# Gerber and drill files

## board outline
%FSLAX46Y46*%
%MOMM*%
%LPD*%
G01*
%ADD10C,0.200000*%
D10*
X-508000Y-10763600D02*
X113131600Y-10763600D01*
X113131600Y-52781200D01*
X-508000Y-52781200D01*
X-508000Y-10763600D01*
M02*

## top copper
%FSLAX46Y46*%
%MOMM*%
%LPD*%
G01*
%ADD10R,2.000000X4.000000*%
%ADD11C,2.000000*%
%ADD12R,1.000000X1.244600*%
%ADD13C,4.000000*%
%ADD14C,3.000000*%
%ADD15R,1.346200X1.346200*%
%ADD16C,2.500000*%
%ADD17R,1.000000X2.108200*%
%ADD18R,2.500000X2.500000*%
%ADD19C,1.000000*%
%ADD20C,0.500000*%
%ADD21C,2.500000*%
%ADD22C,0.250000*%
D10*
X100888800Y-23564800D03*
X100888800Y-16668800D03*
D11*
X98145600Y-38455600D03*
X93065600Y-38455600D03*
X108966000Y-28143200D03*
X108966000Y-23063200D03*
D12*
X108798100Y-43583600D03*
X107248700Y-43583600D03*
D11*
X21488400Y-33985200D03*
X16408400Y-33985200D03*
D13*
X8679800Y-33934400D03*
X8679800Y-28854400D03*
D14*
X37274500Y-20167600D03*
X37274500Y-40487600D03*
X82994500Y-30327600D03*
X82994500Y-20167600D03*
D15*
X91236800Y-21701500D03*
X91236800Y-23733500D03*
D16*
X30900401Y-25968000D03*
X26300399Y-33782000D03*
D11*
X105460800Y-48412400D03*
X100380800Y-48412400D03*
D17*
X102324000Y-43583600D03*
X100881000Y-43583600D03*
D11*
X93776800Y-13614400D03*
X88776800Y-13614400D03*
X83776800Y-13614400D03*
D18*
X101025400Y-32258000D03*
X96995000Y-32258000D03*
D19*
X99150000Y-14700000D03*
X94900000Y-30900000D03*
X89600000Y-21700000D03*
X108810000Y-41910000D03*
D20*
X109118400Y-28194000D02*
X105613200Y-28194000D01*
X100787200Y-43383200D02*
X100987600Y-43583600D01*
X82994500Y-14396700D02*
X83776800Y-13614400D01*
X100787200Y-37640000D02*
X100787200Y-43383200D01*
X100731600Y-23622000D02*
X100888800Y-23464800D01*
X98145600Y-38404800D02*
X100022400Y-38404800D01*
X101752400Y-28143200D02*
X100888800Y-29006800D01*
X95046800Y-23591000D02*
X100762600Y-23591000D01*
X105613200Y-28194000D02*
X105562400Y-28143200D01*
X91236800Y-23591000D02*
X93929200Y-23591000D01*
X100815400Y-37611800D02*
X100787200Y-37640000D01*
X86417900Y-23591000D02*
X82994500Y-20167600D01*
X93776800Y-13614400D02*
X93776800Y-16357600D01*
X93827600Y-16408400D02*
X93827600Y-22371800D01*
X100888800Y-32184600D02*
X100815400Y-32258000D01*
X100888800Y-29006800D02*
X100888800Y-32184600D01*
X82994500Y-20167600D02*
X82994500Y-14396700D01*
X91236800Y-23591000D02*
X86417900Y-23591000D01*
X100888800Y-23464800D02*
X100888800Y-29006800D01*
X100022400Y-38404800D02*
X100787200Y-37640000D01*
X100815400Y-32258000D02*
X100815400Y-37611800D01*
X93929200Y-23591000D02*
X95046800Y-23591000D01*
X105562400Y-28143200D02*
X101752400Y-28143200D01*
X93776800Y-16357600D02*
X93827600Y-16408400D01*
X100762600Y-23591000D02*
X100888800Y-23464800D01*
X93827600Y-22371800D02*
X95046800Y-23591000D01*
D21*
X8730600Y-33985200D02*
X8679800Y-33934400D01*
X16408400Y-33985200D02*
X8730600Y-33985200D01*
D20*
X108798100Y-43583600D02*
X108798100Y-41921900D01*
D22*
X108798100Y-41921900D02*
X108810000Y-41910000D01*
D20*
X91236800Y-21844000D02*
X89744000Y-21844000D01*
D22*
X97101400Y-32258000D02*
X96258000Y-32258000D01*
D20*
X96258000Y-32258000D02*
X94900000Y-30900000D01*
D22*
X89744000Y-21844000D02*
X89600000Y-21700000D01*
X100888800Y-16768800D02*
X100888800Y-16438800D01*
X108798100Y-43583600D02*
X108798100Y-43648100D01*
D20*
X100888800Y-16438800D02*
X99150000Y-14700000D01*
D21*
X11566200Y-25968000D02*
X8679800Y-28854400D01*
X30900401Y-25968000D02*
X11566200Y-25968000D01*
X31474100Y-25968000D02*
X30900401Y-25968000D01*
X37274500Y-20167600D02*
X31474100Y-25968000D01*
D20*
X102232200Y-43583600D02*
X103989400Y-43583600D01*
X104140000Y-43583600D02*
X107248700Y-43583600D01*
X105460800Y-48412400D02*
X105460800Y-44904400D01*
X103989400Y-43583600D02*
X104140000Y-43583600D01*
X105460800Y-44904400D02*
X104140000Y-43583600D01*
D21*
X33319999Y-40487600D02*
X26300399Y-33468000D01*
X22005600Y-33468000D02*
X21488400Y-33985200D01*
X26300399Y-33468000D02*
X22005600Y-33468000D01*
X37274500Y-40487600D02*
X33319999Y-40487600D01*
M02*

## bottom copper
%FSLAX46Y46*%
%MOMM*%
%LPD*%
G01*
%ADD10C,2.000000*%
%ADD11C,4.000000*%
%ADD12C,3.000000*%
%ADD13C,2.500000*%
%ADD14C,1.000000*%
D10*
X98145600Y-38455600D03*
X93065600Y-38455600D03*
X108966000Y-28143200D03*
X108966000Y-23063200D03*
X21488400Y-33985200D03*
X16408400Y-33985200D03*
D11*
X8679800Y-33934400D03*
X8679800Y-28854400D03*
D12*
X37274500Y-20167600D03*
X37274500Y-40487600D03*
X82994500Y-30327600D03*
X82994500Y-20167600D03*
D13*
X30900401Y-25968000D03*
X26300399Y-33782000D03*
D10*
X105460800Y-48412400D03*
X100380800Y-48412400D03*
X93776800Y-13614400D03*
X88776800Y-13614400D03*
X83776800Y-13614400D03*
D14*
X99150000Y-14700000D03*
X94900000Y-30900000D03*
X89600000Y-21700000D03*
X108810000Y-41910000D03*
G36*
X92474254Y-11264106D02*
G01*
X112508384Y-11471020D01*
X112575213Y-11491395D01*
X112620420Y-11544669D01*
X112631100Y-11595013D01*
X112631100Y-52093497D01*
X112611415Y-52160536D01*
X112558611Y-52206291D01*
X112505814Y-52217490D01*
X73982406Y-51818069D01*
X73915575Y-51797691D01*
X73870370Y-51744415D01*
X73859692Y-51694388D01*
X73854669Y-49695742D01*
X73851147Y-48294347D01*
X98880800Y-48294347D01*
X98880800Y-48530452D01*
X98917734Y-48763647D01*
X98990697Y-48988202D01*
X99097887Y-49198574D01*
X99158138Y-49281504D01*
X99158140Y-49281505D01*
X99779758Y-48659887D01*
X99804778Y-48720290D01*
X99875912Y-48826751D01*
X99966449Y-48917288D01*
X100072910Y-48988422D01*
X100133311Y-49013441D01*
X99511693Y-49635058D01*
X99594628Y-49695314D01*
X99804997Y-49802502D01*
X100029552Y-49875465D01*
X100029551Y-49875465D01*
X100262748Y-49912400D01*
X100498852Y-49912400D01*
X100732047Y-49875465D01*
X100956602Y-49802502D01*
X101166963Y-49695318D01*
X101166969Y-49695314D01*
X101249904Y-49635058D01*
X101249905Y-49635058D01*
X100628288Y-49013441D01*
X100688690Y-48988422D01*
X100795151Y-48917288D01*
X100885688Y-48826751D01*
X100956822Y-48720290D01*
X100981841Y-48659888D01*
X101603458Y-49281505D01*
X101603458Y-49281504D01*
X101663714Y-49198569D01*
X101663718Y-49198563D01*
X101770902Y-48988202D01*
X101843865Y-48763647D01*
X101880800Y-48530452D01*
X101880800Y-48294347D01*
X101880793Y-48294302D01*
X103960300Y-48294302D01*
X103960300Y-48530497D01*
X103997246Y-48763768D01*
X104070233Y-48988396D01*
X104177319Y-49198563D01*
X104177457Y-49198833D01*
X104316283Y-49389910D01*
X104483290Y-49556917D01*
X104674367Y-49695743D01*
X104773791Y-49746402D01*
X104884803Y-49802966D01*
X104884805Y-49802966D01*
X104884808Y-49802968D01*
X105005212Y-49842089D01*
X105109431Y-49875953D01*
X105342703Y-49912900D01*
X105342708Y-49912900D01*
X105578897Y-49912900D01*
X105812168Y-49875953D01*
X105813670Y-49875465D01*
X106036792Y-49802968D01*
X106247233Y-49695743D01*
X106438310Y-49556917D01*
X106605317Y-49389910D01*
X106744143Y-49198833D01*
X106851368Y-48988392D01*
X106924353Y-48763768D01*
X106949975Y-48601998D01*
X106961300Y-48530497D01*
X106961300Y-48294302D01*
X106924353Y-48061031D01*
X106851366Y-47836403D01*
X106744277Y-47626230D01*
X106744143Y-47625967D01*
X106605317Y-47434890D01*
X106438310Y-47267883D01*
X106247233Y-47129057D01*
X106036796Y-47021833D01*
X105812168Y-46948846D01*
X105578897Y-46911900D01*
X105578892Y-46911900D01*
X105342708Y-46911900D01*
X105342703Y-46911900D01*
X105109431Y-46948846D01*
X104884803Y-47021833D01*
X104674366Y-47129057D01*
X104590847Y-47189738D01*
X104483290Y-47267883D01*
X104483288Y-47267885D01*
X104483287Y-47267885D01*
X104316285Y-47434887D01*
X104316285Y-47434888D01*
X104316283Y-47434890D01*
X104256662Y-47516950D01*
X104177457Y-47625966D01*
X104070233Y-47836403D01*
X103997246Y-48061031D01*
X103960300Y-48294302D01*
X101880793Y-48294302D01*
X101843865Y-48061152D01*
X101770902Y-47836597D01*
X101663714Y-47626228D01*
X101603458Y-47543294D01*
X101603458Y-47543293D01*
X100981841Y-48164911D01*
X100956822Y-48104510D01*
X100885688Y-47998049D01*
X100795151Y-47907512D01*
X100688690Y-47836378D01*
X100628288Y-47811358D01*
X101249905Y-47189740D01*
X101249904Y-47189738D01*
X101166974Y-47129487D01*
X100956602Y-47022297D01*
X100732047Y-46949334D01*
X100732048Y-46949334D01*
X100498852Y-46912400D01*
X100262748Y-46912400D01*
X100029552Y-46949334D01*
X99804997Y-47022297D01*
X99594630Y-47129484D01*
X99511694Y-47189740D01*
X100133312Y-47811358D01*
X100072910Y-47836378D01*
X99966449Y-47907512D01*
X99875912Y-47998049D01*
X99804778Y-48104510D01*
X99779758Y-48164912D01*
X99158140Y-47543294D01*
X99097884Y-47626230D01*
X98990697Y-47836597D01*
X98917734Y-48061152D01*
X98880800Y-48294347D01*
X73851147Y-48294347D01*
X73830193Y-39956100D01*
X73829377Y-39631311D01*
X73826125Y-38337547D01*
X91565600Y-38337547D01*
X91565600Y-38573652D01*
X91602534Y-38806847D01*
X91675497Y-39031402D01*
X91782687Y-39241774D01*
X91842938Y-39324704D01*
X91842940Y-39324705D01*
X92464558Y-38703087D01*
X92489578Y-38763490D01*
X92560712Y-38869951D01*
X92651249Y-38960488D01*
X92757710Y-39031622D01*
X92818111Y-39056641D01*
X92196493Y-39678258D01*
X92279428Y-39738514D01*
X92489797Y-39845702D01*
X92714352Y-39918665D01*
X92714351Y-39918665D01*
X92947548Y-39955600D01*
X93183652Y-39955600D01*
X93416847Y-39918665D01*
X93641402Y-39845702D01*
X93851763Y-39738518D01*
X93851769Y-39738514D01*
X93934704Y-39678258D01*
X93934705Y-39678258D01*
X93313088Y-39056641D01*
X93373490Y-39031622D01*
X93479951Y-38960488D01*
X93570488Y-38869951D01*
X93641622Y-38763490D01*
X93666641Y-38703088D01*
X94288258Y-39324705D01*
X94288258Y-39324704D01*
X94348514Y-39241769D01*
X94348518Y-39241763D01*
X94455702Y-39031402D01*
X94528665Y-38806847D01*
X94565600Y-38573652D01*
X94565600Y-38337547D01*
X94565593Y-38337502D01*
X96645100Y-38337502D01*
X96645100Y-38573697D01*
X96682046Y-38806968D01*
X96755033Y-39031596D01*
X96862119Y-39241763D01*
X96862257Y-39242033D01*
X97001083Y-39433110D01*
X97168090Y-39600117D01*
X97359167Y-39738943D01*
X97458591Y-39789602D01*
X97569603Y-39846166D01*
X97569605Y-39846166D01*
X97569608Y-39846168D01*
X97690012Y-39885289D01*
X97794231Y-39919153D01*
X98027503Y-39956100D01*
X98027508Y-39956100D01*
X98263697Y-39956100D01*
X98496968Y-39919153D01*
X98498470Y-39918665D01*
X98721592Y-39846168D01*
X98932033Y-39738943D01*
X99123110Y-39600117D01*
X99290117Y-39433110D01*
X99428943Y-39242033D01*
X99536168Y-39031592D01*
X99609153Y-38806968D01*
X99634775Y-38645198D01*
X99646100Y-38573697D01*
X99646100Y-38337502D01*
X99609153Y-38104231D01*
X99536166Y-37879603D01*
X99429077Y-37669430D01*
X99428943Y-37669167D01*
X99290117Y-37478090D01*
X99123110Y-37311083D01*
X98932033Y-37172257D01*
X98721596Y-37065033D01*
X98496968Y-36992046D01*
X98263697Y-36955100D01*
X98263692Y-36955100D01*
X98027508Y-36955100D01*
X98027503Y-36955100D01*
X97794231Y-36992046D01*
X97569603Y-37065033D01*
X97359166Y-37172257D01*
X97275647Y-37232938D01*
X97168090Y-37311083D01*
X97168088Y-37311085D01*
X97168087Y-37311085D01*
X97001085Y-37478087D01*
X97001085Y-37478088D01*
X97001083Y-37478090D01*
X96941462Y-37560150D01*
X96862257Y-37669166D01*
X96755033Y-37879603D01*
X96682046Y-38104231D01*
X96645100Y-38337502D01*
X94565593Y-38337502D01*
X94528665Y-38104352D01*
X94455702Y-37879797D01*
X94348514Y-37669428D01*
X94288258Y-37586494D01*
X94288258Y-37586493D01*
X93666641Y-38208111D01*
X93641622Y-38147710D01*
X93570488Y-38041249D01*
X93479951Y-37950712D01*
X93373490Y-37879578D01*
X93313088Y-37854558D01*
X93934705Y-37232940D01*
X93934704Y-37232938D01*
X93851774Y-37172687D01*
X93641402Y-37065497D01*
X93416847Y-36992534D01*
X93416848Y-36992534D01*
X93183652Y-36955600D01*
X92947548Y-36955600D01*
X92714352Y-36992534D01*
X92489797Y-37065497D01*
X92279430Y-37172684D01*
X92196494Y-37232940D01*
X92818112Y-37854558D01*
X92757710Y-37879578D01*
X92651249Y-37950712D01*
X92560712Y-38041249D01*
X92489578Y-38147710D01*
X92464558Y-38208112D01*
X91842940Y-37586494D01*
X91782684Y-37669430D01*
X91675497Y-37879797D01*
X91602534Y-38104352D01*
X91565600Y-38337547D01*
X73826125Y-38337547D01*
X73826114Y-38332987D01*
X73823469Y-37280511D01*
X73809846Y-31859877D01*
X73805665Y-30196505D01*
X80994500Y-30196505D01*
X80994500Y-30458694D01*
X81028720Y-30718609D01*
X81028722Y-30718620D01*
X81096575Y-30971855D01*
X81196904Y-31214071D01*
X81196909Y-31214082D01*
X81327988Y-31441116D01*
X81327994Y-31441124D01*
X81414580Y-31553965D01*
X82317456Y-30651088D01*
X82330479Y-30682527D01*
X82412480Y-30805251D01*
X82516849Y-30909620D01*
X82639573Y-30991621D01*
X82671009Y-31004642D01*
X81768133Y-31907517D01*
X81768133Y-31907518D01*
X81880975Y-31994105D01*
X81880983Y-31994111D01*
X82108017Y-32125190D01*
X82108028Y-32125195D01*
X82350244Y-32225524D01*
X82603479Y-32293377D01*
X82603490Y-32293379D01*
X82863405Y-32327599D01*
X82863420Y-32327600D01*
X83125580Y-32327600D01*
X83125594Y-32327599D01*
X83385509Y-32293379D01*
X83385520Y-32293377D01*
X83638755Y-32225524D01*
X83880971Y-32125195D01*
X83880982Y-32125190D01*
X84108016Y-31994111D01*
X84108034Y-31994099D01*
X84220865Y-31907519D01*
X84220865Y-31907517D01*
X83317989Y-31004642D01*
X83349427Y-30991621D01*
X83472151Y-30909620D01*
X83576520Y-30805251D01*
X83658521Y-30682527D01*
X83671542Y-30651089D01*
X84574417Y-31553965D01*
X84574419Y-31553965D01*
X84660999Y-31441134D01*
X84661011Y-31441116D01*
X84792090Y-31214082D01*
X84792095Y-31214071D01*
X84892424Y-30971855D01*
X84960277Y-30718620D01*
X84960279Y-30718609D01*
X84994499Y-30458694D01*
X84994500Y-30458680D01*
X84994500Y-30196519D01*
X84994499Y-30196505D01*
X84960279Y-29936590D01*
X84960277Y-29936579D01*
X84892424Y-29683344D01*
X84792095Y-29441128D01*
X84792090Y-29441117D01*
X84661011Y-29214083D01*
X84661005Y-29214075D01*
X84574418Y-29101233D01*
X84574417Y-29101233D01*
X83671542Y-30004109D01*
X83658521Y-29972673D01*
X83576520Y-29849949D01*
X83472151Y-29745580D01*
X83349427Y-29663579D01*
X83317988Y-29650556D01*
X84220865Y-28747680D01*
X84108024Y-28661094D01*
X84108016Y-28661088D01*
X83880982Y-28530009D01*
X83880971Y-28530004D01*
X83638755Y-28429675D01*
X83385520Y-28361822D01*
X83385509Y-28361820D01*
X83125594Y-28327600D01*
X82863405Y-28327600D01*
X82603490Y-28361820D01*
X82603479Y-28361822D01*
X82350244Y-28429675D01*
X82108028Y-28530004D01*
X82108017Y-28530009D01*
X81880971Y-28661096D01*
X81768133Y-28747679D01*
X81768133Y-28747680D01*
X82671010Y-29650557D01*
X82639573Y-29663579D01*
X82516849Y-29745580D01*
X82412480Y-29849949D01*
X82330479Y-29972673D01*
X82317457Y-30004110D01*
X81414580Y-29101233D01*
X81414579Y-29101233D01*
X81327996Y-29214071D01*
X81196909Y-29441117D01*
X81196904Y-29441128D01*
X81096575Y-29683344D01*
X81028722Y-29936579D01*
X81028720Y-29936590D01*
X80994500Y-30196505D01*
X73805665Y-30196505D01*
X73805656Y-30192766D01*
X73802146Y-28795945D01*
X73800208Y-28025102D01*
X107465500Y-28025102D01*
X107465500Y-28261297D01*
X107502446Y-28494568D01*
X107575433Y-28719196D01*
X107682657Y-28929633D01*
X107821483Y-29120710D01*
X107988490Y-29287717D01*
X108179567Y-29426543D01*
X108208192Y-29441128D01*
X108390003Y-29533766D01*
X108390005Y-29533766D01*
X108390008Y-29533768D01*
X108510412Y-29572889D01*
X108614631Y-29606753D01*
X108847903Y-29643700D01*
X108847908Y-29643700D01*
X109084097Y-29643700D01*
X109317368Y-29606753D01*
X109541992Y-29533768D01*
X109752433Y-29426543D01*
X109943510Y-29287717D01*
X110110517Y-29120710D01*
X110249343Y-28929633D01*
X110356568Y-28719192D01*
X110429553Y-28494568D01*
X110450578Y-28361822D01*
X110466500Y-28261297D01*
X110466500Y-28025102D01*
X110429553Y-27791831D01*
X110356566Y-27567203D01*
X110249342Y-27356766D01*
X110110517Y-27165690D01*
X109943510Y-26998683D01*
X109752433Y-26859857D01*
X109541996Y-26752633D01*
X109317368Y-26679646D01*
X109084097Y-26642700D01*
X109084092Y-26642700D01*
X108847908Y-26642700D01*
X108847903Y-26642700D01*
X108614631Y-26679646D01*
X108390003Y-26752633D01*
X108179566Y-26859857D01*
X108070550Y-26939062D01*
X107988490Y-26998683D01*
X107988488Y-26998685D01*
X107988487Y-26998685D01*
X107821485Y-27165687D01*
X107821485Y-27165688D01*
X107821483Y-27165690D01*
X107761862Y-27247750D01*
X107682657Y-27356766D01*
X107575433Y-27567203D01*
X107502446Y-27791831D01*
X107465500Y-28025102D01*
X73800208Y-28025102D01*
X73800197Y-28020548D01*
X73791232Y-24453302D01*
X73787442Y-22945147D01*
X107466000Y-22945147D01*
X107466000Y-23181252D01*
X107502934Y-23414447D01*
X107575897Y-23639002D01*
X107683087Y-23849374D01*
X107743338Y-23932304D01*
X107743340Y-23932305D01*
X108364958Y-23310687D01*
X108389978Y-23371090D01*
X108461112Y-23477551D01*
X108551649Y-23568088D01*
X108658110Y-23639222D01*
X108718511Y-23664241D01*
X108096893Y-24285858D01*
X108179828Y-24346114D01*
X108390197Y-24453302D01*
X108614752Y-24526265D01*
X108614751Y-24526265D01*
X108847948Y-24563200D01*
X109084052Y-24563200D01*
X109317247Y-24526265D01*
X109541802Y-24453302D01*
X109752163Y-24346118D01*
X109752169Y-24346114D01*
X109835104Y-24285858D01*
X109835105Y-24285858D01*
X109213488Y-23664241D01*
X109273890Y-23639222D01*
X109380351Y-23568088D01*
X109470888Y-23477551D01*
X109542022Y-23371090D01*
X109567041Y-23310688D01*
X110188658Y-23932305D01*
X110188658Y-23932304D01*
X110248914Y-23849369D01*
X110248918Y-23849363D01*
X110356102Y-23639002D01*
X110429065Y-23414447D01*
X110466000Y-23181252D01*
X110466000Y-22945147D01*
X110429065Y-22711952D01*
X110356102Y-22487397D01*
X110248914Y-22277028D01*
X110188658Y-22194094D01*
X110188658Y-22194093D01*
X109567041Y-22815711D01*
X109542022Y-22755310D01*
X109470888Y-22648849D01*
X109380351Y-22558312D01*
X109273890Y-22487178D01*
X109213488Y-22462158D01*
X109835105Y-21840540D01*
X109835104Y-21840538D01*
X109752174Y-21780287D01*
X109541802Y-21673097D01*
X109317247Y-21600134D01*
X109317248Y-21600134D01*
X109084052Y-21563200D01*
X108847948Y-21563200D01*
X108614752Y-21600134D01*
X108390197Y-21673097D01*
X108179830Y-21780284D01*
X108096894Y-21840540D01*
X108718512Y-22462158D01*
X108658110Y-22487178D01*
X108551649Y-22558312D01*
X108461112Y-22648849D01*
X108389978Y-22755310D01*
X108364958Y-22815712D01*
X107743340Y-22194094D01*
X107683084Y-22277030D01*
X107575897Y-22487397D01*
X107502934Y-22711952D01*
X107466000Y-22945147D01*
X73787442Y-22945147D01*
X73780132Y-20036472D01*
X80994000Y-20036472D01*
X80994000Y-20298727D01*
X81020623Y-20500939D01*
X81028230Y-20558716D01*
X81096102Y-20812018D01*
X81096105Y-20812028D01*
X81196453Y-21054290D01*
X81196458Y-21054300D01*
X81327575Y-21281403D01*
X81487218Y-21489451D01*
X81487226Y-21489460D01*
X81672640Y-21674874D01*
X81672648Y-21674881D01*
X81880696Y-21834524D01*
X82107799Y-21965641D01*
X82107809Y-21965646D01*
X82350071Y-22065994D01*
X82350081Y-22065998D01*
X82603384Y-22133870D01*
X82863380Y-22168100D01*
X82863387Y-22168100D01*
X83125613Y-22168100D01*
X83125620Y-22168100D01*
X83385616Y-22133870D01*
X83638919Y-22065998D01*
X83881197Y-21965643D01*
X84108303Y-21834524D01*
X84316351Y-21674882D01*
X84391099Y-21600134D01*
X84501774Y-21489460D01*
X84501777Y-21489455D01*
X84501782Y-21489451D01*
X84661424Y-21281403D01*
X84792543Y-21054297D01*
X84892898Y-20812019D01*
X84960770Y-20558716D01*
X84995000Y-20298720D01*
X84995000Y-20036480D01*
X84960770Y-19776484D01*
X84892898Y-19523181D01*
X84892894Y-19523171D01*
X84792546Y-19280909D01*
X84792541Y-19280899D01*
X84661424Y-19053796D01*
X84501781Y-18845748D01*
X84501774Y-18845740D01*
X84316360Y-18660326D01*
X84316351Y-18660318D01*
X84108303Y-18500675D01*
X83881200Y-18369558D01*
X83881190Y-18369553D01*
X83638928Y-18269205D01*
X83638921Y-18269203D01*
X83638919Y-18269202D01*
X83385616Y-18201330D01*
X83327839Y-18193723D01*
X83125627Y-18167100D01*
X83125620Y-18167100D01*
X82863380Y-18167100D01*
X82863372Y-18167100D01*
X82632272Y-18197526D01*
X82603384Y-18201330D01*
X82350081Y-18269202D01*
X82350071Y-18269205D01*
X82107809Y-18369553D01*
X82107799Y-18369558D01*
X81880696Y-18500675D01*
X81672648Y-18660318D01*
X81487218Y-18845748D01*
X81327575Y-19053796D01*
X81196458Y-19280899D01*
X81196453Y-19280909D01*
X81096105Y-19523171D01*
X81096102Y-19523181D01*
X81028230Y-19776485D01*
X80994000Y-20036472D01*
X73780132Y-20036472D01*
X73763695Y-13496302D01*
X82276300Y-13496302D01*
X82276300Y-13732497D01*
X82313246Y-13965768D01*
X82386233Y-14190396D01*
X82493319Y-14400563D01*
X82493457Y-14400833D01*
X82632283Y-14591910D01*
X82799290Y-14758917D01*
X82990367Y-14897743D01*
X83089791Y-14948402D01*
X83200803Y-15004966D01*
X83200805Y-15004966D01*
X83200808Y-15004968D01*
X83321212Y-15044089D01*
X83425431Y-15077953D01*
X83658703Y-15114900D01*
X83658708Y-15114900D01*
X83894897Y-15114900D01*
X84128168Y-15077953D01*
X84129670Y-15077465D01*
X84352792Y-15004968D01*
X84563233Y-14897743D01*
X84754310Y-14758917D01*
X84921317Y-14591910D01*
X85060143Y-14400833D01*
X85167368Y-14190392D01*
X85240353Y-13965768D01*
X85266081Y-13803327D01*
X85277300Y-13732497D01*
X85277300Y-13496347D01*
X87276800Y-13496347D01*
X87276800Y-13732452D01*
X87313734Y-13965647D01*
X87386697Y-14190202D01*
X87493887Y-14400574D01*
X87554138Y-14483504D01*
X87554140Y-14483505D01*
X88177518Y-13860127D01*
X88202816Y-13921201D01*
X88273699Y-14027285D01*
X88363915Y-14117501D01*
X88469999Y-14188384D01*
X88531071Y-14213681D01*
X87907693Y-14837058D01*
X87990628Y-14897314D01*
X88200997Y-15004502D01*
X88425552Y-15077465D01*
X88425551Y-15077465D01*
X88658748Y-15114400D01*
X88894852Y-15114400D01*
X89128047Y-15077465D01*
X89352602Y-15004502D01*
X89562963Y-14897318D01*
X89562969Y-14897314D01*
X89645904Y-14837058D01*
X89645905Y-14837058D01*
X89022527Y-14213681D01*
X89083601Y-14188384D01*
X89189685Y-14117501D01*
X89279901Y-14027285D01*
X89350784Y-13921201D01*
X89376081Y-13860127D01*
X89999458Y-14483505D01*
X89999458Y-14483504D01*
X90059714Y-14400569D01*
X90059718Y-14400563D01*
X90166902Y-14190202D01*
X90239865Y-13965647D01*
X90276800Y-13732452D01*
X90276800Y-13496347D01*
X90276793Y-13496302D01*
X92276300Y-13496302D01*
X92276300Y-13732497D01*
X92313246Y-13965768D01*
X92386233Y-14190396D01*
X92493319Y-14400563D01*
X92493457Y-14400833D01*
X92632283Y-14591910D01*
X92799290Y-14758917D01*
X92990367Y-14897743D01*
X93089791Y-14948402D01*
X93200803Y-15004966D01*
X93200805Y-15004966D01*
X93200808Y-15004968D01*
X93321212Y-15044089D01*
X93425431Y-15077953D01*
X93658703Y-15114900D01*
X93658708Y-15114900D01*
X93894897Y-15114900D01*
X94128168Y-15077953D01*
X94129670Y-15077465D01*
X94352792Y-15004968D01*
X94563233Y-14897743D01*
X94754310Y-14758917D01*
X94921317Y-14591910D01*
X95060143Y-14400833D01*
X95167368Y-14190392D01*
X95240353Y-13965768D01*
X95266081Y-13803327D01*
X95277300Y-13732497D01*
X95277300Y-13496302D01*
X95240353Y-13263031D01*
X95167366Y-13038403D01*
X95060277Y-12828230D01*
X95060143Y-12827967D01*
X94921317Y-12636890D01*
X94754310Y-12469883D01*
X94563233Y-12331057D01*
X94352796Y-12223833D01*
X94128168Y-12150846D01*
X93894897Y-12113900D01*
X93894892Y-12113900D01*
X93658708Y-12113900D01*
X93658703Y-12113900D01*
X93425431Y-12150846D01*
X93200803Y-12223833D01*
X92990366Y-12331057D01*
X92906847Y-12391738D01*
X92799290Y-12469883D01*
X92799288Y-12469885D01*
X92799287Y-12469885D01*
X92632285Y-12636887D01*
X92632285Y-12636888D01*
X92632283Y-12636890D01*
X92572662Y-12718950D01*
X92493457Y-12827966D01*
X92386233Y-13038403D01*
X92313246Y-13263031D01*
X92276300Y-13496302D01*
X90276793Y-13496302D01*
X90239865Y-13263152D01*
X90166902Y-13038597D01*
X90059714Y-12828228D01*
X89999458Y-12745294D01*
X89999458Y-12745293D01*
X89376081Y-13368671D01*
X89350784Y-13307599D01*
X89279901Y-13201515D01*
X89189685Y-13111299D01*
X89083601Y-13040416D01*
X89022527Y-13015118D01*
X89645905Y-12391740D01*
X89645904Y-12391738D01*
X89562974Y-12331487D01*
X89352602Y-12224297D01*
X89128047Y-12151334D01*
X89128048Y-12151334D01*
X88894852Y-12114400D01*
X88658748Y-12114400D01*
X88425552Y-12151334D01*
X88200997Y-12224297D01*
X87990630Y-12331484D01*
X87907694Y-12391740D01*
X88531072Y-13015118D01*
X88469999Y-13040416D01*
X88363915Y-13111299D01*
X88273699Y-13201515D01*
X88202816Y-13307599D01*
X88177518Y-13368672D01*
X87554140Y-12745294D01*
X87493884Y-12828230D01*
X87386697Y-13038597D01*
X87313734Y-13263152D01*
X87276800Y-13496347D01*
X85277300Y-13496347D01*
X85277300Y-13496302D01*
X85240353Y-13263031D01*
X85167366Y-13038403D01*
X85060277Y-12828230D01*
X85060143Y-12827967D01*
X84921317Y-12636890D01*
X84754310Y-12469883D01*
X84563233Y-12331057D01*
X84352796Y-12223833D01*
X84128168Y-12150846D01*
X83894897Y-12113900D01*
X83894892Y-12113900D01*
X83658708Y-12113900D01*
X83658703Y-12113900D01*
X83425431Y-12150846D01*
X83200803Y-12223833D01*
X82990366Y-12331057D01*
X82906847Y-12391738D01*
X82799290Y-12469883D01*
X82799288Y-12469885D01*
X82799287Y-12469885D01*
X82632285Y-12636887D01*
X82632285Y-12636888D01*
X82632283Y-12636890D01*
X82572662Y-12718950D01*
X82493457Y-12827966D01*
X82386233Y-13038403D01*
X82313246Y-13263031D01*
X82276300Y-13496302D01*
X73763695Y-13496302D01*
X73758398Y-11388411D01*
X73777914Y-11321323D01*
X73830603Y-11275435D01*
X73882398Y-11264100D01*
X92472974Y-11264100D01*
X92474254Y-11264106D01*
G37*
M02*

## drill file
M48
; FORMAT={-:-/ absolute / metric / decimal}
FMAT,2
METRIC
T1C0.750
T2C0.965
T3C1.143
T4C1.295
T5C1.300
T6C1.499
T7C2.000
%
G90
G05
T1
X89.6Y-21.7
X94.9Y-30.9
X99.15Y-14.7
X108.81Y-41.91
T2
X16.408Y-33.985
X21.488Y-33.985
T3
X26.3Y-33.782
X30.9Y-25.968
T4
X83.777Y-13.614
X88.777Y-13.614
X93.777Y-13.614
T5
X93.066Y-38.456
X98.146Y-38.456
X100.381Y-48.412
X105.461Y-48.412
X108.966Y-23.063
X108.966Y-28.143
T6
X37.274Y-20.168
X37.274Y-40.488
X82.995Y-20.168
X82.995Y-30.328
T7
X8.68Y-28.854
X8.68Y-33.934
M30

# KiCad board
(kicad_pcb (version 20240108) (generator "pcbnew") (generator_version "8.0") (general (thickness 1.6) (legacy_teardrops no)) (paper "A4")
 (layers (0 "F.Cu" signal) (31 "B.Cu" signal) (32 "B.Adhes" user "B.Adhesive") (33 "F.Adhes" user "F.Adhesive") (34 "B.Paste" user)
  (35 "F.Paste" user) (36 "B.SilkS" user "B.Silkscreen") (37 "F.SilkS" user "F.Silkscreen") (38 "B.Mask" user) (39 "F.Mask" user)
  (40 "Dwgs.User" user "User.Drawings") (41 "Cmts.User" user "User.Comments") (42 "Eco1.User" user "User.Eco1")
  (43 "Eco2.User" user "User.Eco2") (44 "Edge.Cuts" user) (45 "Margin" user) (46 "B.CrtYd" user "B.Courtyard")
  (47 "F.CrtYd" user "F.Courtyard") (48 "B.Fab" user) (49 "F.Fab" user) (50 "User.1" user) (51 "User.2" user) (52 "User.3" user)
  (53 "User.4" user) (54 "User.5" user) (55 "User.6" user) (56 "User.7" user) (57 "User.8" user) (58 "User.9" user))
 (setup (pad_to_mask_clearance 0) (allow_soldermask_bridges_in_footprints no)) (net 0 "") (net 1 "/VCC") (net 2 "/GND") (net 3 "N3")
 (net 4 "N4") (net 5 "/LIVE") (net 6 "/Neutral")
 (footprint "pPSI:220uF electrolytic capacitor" (layer "F.Cu") (at 100.8888 20.1168 90)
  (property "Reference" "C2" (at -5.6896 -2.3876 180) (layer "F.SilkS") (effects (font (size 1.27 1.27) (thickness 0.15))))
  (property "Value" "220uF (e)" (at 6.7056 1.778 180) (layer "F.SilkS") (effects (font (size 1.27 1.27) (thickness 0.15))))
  (pad "1" smd rect (at -3.448 0 90) (size 4 2) (layers "F.Cu" "F.Paste" "F.Mask") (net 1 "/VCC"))
  (pad "2" smd rect (at 3.448 0 90) (size 4 2) (layers "F.Cu" "F.Paste" "F.Mask") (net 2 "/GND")))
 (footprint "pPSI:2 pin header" (layer "F.Cu") (at 98.1456 38.4556 180)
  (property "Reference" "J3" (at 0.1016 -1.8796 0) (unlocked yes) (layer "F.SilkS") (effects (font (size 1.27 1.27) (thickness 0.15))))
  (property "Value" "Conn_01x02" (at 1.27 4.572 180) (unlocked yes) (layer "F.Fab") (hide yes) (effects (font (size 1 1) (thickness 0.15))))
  (pad "1" thru_hole circle (at 0 0 180) (size 2 2) (drill 1.3) (layers "*.Cu" "*.Mask") (remove_unused_layers no) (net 1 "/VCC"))
  (pad "2" thru_hole circle (at 5.08 0 180) (size 2 2) (drill 1.3) (layers "*.Cu" "*.Mask") (remove_unused_layers no) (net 2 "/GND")))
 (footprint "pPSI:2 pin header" (layer "F.Cu") (at 108.966 28.1432 90)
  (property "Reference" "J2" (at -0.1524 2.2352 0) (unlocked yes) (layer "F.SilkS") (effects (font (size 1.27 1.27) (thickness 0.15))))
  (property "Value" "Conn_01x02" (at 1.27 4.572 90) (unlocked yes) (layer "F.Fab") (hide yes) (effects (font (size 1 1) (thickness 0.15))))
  (pad "1" thru_hole circle (at 0 0 90) (size 2 2) (drill 1.3) (layers "*.Cu" "*.Mask") (remove_unused_layers no) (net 1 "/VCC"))
  (pad "2" thru_hole circle (at 5.08 0 90) (size 2 2) (drill 1.3) (layers "*.Cu" "*.Mask") (remove_unused_layers no) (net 2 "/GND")))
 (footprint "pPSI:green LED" (layer "F.Cu") (at 108.0234 43.5836 180)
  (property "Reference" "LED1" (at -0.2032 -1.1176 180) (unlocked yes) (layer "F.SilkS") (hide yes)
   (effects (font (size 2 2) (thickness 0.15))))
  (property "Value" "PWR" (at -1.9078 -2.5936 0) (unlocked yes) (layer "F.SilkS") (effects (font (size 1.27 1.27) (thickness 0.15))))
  (pad "1" smd rect (at -0.7747 0 180) (size 1 1.2446) (layers "F.Cu" "F.Paste" "F.Mask") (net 2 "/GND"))
  (pad "2" smd rect (at 0.7747 0 180) (size 1 1.2446) (layers "F.Cu" "F.Paste" "F.Mask") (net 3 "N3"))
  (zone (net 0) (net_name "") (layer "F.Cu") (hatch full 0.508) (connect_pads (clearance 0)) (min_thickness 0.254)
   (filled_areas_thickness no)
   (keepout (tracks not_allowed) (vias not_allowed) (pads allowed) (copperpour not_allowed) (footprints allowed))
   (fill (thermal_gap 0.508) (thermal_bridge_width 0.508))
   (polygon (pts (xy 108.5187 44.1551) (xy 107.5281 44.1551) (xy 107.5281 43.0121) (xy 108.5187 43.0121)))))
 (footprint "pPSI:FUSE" (layer "F.Cu") (at 21.4884 33.9852 180)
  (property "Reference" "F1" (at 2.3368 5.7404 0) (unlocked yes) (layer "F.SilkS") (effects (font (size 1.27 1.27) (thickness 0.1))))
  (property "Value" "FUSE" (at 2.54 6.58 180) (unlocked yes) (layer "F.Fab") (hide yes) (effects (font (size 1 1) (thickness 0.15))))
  (pad "1" thru_hole circle (at 0 0 180) (size 2 2) (drill 0.9652) (layers "*.Cu" "*.Mask") (remove_unused_layers no) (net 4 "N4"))
  (pad "2" thru_hole circle (at 5.08 0 180) (size 2 2) (drill 0.9652) (layers "*.Cu" "*.Mask") (remove_unused_layers no) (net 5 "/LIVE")))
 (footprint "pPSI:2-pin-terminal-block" (layer "F.Cu") (at 8.6798 33.9344 90)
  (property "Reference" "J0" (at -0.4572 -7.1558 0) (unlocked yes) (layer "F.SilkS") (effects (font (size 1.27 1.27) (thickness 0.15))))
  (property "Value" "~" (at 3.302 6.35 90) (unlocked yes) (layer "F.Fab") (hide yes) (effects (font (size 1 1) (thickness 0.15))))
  (pad "1" thru_hole circle (at 0 0 90) (size 4 4) (drill 2) (layers "*.Cu" "*.Mask") (remove_unused_layers no) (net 5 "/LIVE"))
  (pad "2" thru_hole circle (at 5.08 0 90) (size 4 4) (drill 2) (layers "*.Cu" "*.Mask") (remove_unused_layers no) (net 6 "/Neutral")))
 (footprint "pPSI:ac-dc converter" (layer "F.Cu") (at 37.2745 20.1676)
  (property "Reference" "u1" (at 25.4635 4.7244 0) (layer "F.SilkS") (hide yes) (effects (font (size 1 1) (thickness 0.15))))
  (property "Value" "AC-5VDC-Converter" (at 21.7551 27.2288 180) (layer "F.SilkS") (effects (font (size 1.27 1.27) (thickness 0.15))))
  (pad "1" thru_hole circle (at 0 0) (size 3 3) (drill 1.4986) (layers "*.Cu" "*.Mask") (remove_unused_layers no) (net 6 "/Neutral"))
  (pad "2" thru_hole circle (at 0 20.32) (size 3 3) (drill 1.4986) (layers "*.Cu" "*.Mask") (remove_unused_layers no) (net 4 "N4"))
  (pad "3" thru_hole circle (at 45.72 10.16) (size 3 3) (drill 1.4986) (layers "*.Cu" "*.Mask") (remove_unused_layers no) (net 2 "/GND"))
  (pad "4" thru_hole circle (at 45.72 0) (size 3 3) (drill 1.4986) (layers "*.Cu" "*.Mask") (remove_unused_layers no) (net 1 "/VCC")))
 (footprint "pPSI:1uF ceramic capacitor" (layer "F.Cu") (at 91.2368 22.7175 -90)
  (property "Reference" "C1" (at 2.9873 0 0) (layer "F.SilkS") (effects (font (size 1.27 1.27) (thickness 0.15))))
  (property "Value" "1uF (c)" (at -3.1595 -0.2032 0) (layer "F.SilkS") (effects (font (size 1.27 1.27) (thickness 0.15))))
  (pad "1" smd rect (at -1.016 0 270) (size 1.3462 1.3462) (layers "F.Cu" "F.Paste" "F.Mask") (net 2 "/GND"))
  (pad "2" smd rect (at 1.016 0 270) (size 1.3462 1.3462) (layers "F.Cu" "F.Paste" "F.Mask") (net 1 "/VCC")))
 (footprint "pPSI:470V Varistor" (layer "F.Cu") (at 28.6004 29.718 -90)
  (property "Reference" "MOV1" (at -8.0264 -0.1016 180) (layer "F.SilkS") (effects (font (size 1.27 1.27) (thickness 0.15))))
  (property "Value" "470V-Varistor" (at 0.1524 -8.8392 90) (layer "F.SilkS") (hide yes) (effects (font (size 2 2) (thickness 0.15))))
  (pad "1" thru_hole circle (at -3.75 -2.300001 270) (size 2.5 2.5) (drill 1.143) (layers "*.Cu" "*.Mask") (remove_unused_layers no)
   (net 6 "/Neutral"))
  (pad "2" thru_hole circle (at 4.064 2.300001 270) (size 2.5 2.5) (drill 1.143) (layers "*.Cu" "*.Mask") (remove_unused_layers no)
   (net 4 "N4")))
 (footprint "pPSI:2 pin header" (layer "F.Cu") (at 105.4608 48.4124 180)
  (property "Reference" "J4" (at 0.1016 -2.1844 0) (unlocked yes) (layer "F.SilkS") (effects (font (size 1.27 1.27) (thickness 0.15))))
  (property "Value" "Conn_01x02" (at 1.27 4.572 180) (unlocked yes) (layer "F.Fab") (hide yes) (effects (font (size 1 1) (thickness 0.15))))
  (pad "1" thru_hole circle (at 0 0 180) (size 2 2) (drill 1.3) (layers "*.Cu" "*.Mask") (remove_unused_layers no) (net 3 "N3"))
  (pad "2" thru_hole circle (at 5.08 0 180) (size 2 2) (drill 1.3) (layers "*.Cu" "*.Mask") (remove_unused_layers no) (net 2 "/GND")))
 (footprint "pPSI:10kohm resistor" (layer "F.Cu") (at 101.6099 43.5836 180)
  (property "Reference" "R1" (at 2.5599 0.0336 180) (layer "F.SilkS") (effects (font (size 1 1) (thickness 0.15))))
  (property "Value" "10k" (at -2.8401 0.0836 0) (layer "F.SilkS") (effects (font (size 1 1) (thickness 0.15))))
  (pad "1" smd rect (at -0.7141 0 180) (size 1 2.1082) (layers "F.Cu" "F.Paste" "F.Mask") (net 3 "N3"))
  (pad "2" smd rect (at 0.7289 0 180) (size 1 2.1082) (layers "F.Cu" "F.Paste" "F.Mask") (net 1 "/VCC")))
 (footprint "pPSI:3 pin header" (layer "F.Cu") (at 93.7768 13.6144 180)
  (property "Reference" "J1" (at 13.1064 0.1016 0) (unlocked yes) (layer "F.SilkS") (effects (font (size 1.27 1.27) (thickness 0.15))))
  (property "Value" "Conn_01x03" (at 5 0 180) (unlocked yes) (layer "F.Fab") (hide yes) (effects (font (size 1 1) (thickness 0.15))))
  (pad "1" thru_hole circle (at 0 0 180) (size 2 2) (drill 1.2954) (layers "*.Cu" "*.Mask") (remove_unused_layers no) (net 1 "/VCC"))
  (pad "2" thru_hole circle (at 5 0 180) (size 2 2) (drill 1.2954) (layers "*.Cu" "*.Mask") (remove_unused_layers no) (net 2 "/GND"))
  (pad "3" thru_hole circle (at 10 0 180) (size 2 2) (drill 1.2954) (layers "*.Cu" "*.Mask") (remove_unused_layers no) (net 1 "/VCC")))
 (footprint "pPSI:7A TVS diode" (layer "F.Cu") (at 98.9584 32.258 180)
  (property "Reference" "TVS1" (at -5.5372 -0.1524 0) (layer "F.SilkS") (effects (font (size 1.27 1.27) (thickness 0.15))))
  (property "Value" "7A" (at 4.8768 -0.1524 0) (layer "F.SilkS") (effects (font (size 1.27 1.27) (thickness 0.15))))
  (pad "1" smd rect (at -2.067 0 270) (size 2.5 2.5) (layers "F.Cu" "F.Paste" "F.Mask") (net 1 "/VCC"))
  (pad "2" smd rect (at 1.9634 0 270) (size 2.5 2.5) (layers "F.Cu" "F.Paste" "F.Mask") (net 2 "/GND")))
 (gr_rect (start -0.508 10.7636) (end 113.1316 52.7812) (stroke (width 0.2) (type default)) (fill none) (layer "Edge.Cuts"))
 (segment (start 109.1184 28.194) (end 105.6132 28.194) (width 0.5) (layer "F.Cu") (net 1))
 (segment (start 100.7872 43.3832) (end 100.9876 43.5836) (width 0.5) (layer "F.Cu") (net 1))
 (segment (start 82.9945 14.3967) (end 83.7768 13.6144) (width 0.5) (layer "F.Cu") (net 1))
 (segment (start 100.7872 37.64) (end 100.7872 43.3832) (width 0.5) (layer "F.Cu") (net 1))
 (segment (start 100.7316 23.622) (end 100.8888 23.4648) (width 0.5) (layer "F.Cu") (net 1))
 (segment (start 98.1456 38.4048) (end 100.0224 38.4048) (width 0.5) (layer "F.Cu") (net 1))
 (segment (start 101.7524 28.1432) (end 100.8888 29.0068) (width 0.5) (layer "F.Cu") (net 1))
 (segment (start 95.0468 23.591) (end 100.7626 23.591) (width 0.5) (layer "F.Cu") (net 1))
 (segment (start 105.6132 28.194) (end 105.5624 28.1432) (width 0.5) (layer "F.Cu") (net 1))
 (segment (start 91.2368 23.591) (end 93.9292 23.591) (width 0.5) (layer "F.Cu") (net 1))
 (segment (start 100.8154 37.6118) (end 100.7872 37.64) (width 0.5) (layer "F.Cu") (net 1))
 (segment (start 86.4179 23.591) (end 82.9945 20.1676) (width 0.5) (layer "F.Cu") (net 1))
 (segment (start 93.7768 13.6144) (end 93.7768 16.3576) (width 0.5) (layer "F.Cu") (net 1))
 (segment (start 93.8276 16.4084) (end 93.8276 22.3718) (width 0.5) (layer "F.Cu") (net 1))
 (segment (start 100.8888 32.1846) (end 100.8154 32.258) (width 0.5) (layer "F.Cu") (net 1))
 (segment (start 100.8888 29.0068) (end 100.8888 32.1846) (width 0.5) (layer "F.Cu") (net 1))
 (segment (start 82.9945 20.1676) (end 82.9945 14.3967) (width 0.5) (layer "F.Cu") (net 1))
 (segment (start 91.2368 23.591) (end 86.4179 23.591) (width 0.5) (layer "F.Cu") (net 1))
 (segment (start 100.8888 23.4648) (end 100.8888 29.0068) (width 0.5) (layer "F.Cu") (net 1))
 (segment (start 100.0224 38.4048) (end 100.7872 37.64) (width 0.5) (layer "F.Cu") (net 1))
 (segment (start 100.8154 32.258) (end 100.8154 37.6118) (width 0.5) (layer "F.Cu") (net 1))
 (segment (start 93.9292 23.591) (end 95.0468 23.591) (width 0.5) (layer "F.Cu") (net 1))
 (segment (start 105.5624 28.1432) (end 101.7524 28.1432) (width 0.5) (layer "F.Cu") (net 1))
 (segment (start 93.7768 16.3576) (end 93.8276 16.4084) (width 0.5) (layer "F.Cu") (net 1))
 (segment (start 100.7626 23.591) (end 100.8888 23.4648) (width 0.5) (layer "F.Cu") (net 1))
 (segment (start 93.8276 22.3718) (end 95.0468 23.591) (width 0.5) (layer "F.Cu") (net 1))
 (segment (start 8.7306 33.9852) (end 8.6798 33.9344) (width 2.5) (layer "F.Cu") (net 5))
 (segment (start 16.4084 33.9852) (end 8.7306 33.9852) (width 2.5) (layer "F.Cu") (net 5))
 (segment (start 108.7981 43.5836) (end 108.7981 41.9219) (width 0.5) (layer "F.Cu") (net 2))
 (segment (start 108.7981 41.9219) (end 108.81 41.91) (width 0.25) (layer "F.Cu") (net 2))
 (segment (start 91.2368 21.844) (end 89.744 21.844) (width 0.5) (layer "F.Cu") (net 2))
 (segment (start 97.1014 32.258) (end 96.258 32.258) (width 0.25) (layer "F.Cu") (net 2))
 (segment (start 96.258 32.258) (end 94.9 30.9) (width 0.5) (layer "F.Cu") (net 2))
 (segment (start 89.744 21.844) (end 89.6 21.7) (width 0.25) (layer "F.Cu") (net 2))
 (segment (start 100.8888 16.7688) (end 100.8888 16.4388) (width 0.25) (layer "F.Cu") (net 2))
 (segment (start 108.7981 43.5836) (end 108.7981 43.6481) (width 0.25) (layer "F.Cu") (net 2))
 (segment (start 100.8888 16.4388) (end 99.15 14.7) (width 0.5) (layer "F.Cu") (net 2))
 (via blind (at 99.15 14.7) (size 1) (drill 0.75) (layers "F.Cu" "B.Cu") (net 2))
 (via blind (at 94.9 30.9) (size 1) (drill 0.75) (layers "F.Cu" "B.Cu") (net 2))
 (via blind (at 89.6 21.7) (size 1) (drill 0.75) (layers "F.Cu" "B.Cu") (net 2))
 (via blind (at 108.81 41.91) (size 1) (drill 0.75) (layers "F.Cu" "B.Cu") (free yes) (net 2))
 (segment (start 11.5662 25.968) (end 8.6798 28.8544) (width 2.5) (layer "F.Cu") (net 6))
 (segment (start 30.900401 25.968) (end 11.5662 25.968) (width 2.5) (layer "F.Cu") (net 6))
 (segment (start 31.4741 25.968) (end 30.900401 25.968) (width 2.5) (layer "F.Cu") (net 6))
 (segment (start 37.2745 20.1676) (end 31.4741 25.968) (width 2.5) (layer "F.Cu") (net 6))
 (segment (start 102.2322 43.5836) (end 103.9894 43.5836) (width 0.5) (layer "F.Cu") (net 3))
 (segment (start 104.14 43.5836) (end 107.2487 43.5836) (width 0.5) (layer "F.Cu") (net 3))
 (segment (start 105.4608 48.4124) (end 105.4608 44.9044) (width 0.5) (layer "F.Cu") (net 3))
 (segment (start 103.9894 43.5836) (end 104.14 43.5836) (width 0.5) (layer "F.Cu") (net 3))
 (segment (start 105.4608 44.9044) (end 104.14 43.5836) (width 0.5) (layer "F.Cu") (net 3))
 (segment (start 33.319999 40.4876) (end 26.300399 33.468) (width 2.5) (layer "F.Cu") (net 4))
 (segment (start 22.0056 33.468) (end 21.4884 33.9852) (width 2.5) (layer "F.Cu") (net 4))
 (segment (start 26.300399 33.468) (end 22.0056 33.468) (width 2.5) (layer "F.Cu") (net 4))
 (segment (start 37.2745 40.4876) (end 33.319999 40.4876) (width 2.5) (layer "F.Cu") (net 4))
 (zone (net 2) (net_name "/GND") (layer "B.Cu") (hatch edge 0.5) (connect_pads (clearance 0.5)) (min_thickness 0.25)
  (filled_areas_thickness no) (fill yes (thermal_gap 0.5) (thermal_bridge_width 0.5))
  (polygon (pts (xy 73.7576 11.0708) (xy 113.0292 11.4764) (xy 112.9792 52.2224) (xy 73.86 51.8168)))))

